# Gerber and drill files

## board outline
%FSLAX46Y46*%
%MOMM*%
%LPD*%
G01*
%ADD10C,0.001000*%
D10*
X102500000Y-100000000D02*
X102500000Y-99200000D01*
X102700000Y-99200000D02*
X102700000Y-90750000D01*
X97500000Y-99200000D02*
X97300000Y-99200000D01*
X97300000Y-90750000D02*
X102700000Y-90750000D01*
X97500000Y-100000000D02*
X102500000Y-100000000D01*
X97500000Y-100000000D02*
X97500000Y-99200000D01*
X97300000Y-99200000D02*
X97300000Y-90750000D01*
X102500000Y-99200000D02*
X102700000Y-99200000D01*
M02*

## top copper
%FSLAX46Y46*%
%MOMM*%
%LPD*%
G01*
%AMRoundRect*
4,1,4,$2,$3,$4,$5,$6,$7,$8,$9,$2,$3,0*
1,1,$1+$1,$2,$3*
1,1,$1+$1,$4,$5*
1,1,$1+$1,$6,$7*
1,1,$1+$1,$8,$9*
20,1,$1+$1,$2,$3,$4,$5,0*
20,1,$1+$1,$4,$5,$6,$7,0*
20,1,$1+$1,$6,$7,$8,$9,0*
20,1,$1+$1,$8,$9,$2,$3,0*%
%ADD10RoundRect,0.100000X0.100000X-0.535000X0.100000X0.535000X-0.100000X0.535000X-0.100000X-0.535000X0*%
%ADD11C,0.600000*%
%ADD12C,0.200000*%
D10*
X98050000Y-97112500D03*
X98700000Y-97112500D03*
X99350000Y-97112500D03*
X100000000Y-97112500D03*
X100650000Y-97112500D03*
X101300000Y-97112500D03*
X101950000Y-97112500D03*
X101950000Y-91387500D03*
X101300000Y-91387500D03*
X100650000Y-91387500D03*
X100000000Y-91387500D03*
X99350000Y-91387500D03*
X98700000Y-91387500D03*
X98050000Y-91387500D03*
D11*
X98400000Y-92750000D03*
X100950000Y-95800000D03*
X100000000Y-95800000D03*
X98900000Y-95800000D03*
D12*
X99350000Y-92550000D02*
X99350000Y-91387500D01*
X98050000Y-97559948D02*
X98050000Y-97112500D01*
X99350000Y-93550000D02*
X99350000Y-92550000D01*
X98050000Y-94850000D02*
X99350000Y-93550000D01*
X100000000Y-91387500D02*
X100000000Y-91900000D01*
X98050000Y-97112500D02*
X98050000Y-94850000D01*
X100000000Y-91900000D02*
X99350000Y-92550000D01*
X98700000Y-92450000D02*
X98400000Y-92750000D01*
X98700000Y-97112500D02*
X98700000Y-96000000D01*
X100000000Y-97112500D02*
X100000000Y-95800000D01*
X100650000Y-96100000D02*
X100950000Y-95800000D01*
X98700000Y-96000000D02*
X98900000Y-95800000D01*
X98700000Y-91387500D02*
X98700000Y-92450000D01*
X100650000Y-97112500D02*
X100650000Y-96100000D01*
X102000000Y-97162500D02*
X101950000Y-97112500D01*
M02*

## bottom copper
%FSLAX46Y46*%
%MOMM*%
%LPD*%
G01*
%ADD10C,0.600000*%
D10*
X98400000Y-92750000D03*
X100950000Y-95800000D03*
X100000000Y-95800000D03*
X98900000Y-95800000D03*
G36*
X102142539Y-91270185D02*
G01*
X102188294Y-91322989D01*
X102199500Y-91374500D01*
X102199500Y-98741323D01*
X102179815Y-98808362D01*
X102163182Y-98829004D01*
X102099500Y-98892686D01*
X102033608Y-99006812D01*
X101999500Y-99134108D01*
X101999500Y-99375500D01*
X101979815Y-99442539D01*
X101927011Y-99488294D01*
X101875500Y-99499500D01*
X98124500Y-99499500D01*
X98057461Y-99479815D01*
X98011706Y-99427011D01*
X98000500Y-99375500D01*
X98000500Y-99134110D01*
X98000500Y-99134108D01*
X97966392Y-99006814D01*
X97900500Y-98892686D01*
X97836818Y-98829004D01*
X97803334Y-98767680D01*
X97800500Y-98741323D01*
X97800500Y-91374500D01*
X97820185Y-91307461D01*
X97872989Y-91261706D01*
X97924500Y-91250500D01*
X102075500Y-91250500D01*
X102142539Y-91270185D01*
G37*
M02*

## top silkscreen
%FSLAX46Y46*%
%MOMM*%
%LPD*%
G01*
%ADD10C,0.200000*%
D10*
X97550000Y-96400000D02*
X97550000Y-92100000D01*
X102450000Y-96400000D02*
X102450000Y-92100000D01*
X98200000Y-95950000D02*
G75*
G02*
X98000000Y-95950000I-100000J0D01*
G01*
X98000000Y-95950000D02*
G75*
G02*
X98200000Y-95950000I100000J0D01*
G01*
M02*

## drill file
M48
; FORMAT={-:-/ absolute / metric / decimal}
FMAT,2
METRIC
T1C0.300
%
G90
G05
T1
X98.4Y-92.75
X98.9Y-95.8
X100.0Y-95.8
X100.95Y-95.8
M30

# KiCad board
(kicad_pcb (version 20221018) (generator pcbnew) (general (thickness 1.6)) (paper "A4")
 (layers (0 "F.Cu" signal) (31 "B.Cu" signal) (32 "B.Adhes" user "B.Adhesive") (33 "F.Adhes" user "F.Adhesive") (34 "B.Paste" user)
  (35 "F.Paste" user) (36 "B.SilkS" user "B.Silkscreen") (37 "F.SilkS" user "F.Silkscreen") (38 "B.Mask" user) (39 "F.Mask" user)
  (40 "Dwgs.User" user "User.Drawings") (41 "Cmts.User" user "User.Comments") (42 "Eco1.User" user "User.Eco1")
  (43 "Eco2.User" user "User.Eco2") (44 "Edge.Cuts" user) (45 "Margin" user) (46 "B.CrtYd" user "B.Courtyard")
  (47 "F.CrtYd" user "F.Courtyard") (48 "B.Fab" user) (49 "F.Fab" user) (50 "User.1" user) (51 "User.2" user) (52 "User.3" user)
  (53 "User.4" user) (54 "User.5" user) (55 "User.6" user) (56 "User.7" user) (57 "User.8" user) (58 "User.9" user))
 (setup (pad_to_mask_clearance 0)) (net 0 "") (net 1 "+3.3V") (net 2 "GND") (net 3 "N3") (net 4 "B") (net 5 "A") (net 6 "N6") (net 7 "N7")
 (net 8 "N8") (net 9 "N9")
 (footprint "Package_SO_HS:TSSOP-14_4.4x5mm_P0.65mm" (layer "F.Cu") (at 100 94.25 90)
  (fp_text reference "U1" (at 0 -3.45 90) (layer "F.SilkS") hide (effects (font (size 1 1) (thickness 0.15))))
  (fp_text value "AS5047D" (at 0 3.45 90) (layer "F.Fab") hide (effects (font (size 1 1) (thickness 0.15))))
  (fp_line (start -2.15 -2.45) (end 2.15 -2.45) (stroke (width 0.2) (type default)) (layer "F.SilkS"))
  (fp_line (start -2.15 2.45) (end 2.15 2.45) (stroke (width 0.2) (type default)) (layer "F.SilkS"))
  (fp_circle (center -1.7 -1.9) (end -1.7 -1.8) (stroke (width 0.2) (type default)) (fill none) (layer "F.SilkS"))
  (pad "1" smd roundrect (at -2.8625 -1.95 90) (size 1.27 0.4) (layers "F.Cu" "F.Paste" "F.Mask") (roundrect_rratio 0.25) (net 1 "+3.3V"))
  (pad "2" smd roundrect (at -2.8625 -1.3 90) (size 1.27 0.4) (layers "F.Cu" "F.Paste" "F.Mask") (roundrect_rratio 0.25) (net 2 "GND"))
  (pad "3" smd roundrect (at -2.8625 -0.65 90) (size 1.27 0.4) (layers "F.Cu" "F.Paste" "F.Mask") (roundrect_rratio 0.25) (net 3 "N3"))
  (pad "4" smd roundrect (at -2.8625 0 90) (size 1.27 0.4) (layers "F.Cu" "F.Paste" "F.Mask") (roundrect_rratio 0.25) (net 2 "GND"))
  (pad "5" smd roundrect (at -2.8625 0.65 90) (size 1.27 0.4) (layers "F.Cu" "F.Paste" "F.Mask") (roundrect_rratio 0.25) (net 2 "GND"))
  (pad "6" smd roundrect (at -2.8625 1.3 90) (size 1.27 0.4) (layers "F.Cu" "F.Paste" "F.Mask") (roundrect_rratio 0.25) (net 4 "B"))
  (pad "7" smd roundrect (at -2.8625 1.95 90) (size 1.27 0.4) (layers "F.Cu" "F.Paste" "F.Mask") (roundrect_rratio 0.25) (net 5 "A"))
  (pad "8" smd roundrect (at 2.8625 1.95 90) (size 1.27 0.4) (layers "F.Cu" "F.Paste" "F.Mask") (roundrect_rratio 0.25) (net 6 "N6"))
  (pad "9" smd roundrect (at 2.8625 1.3 90) (size 1.27 0.4) (layers "F.Cu" "F.Paste" "F.Mask") (roundrect_rratio 0.25) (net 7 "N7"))
  (pad "10" smd roundrect (at 2.8625 0.65 90) (size 1.27 0.4) (layers "F.Cu" "F.Paste" "F.Mask") (roundrect_rratio 0.25) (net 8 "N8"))
  (pad "11" smd roundrect (at 2.8625 0 90) (size 1.27 0.4) (layers "F.Cu" "F.Paste" "F.Mask") (roundrect_rratio 0.25) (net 1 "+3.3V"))
  (pad "12" smd roundrect (at 2.8625 -0.65 90) (size 1.27 0.4) (layers "F.Cu" "F.Paste" "F.Mask") (roundrect_rratio 0.25) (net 1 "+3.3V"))
  (pad "13" smd roundrect (at 2.8625 -1.3 90) (size 1.27 0.4) (layers "F.Cu" "F.Paste" "F.Mask") (roundrect_rratio 0.25) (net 2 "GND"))
  (pad "14" smd roundrect (at 2.8625 -1.95 90) (size 1.27 0.4) (layers "F.Cu" "F.Paste" "F.Mask") (roundrect_rratio 0.25) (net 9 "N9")))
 (gr_line (start 102.5 100) (end 102.5 99.2) (stroke (width 0.001) (type solid)) (layer "Edge.Cuts"))
 (gr_line (start 102.7 99.2) (end 102.7 90.75) (stroke (width 0.001) (type solid)) (layer "Edge.Cuts"))
 (gr_line (start 97.5 99.2) (end 97.3 99.2) (stroke (width 0.001) (type solid)) (layer "Edge.Cuts"))
 (gr_line (start 97.3 90.75) (end 102.7 90.75) (stroke (width 0.001) (type solid)) (layer "Edge.Cuts"))
 (gr_line (start 97.5 100) (end 102.5 100) (stroke (width 0.001) (type solid)) (layer "Edge.Cuts"))
 (gr_line (start 97.5 100) (end 97.5 99.2) (stroke (width 0.001) (type solid)) (layer "Edge.Cuts"))
 (gr_line (start 97.3 99.2) (end 97.3 90.75) (stroke (width 0.001) (type solid)) (layer "Edge.Cuts"))
 (gr_line (start 102.5 99.2) (end 102.7 99.2) (stroke (width 0.001) (type solid)) (layer "Edge.Cuts"))
 (segment (start 99.35 92.55) (end 99.35 91.3875) (width 0.2) (layer "F.Cu") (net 1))
 (segment (start 98.05 97.559948) (end 98.05 97.1125) (width 0.2) (layer "F.Cu") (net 1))
 (segment (start 99.35 93.55) (end 99.35 92.55) (width 0.2) (layer "F.Cu") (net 1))
 (segment (start 98.05 94.85) (end 99.35 93.55) (width 0.2) (layer "F.Cu") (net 1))
 (segment (start 100 91.3875) (end 100 91.9) (width 0.2) (layer "F.Cu") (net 1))
 (segment (start 98.05 97.1125) (end 98.05 94.85) (width 0.2) (layer "F.Cu") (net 1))
 (segment (start 100 91.9) (end 99.35 92.55) (width 0.2) (layer "F.Cu") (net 1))
 (segment (start 98.7 92.45) (end 98.4 92.75) (width 0.2) (layer "F.Cu") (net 2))
 (segment (start 98.7 97.1125) (end 98.7 96) (width 0.2) (layer "F.Cu") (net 2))
 (segment (start 100 97.1125) (end 100 95.8) (width 0.2) (layer "F.Cu") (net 2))
 (segment (start 100.65 96.1) (end 100.95 95.8) (width 0.2) (layer "F.Cu") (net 2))
 (segment (start 98.7 96) (end 98.9 95.8) (width 0.2) (layer "F.Cu") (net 2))
 (segment (start 98.7 91.3875) (end 98.7 92.45) (width 0.2) (layer "F.Cu") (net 2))
 (segment (start 100.65 97.1125) (end 100.65 96.1) (width 0.2) (layer "F.Cu") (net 2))
 (via (at 98.4 92.75) (size 0.6) (drill 0.3) (layers "F.Cu" "B.Cu") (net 2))
 (via (at 100.95 95.8) (size 0.6) (drill 0.3) (layers "F.Cu" "B.Cu") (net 2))
 (via (at 100 95.8) (size 0.6) (drill 0.3) (layers "F.Cu" "B.Cu") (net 2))
 (via (at 98.9 95.8) (size 0.6) (drill 0.3) (layers "F.Cu" "B.Cu") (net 2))
 (segment (start 102 97.1625) (end 101.95 97.1125) (width 0.2) (layer "F.Cu") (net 5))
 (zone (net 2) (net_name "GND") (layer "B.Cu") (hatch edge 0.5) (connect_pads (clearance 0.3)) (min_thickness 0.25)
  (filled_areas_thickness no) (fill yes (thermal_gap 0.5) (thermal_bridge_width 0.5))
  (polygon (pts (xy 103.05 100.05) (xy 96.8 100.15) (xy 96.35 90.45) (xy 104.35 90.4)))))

